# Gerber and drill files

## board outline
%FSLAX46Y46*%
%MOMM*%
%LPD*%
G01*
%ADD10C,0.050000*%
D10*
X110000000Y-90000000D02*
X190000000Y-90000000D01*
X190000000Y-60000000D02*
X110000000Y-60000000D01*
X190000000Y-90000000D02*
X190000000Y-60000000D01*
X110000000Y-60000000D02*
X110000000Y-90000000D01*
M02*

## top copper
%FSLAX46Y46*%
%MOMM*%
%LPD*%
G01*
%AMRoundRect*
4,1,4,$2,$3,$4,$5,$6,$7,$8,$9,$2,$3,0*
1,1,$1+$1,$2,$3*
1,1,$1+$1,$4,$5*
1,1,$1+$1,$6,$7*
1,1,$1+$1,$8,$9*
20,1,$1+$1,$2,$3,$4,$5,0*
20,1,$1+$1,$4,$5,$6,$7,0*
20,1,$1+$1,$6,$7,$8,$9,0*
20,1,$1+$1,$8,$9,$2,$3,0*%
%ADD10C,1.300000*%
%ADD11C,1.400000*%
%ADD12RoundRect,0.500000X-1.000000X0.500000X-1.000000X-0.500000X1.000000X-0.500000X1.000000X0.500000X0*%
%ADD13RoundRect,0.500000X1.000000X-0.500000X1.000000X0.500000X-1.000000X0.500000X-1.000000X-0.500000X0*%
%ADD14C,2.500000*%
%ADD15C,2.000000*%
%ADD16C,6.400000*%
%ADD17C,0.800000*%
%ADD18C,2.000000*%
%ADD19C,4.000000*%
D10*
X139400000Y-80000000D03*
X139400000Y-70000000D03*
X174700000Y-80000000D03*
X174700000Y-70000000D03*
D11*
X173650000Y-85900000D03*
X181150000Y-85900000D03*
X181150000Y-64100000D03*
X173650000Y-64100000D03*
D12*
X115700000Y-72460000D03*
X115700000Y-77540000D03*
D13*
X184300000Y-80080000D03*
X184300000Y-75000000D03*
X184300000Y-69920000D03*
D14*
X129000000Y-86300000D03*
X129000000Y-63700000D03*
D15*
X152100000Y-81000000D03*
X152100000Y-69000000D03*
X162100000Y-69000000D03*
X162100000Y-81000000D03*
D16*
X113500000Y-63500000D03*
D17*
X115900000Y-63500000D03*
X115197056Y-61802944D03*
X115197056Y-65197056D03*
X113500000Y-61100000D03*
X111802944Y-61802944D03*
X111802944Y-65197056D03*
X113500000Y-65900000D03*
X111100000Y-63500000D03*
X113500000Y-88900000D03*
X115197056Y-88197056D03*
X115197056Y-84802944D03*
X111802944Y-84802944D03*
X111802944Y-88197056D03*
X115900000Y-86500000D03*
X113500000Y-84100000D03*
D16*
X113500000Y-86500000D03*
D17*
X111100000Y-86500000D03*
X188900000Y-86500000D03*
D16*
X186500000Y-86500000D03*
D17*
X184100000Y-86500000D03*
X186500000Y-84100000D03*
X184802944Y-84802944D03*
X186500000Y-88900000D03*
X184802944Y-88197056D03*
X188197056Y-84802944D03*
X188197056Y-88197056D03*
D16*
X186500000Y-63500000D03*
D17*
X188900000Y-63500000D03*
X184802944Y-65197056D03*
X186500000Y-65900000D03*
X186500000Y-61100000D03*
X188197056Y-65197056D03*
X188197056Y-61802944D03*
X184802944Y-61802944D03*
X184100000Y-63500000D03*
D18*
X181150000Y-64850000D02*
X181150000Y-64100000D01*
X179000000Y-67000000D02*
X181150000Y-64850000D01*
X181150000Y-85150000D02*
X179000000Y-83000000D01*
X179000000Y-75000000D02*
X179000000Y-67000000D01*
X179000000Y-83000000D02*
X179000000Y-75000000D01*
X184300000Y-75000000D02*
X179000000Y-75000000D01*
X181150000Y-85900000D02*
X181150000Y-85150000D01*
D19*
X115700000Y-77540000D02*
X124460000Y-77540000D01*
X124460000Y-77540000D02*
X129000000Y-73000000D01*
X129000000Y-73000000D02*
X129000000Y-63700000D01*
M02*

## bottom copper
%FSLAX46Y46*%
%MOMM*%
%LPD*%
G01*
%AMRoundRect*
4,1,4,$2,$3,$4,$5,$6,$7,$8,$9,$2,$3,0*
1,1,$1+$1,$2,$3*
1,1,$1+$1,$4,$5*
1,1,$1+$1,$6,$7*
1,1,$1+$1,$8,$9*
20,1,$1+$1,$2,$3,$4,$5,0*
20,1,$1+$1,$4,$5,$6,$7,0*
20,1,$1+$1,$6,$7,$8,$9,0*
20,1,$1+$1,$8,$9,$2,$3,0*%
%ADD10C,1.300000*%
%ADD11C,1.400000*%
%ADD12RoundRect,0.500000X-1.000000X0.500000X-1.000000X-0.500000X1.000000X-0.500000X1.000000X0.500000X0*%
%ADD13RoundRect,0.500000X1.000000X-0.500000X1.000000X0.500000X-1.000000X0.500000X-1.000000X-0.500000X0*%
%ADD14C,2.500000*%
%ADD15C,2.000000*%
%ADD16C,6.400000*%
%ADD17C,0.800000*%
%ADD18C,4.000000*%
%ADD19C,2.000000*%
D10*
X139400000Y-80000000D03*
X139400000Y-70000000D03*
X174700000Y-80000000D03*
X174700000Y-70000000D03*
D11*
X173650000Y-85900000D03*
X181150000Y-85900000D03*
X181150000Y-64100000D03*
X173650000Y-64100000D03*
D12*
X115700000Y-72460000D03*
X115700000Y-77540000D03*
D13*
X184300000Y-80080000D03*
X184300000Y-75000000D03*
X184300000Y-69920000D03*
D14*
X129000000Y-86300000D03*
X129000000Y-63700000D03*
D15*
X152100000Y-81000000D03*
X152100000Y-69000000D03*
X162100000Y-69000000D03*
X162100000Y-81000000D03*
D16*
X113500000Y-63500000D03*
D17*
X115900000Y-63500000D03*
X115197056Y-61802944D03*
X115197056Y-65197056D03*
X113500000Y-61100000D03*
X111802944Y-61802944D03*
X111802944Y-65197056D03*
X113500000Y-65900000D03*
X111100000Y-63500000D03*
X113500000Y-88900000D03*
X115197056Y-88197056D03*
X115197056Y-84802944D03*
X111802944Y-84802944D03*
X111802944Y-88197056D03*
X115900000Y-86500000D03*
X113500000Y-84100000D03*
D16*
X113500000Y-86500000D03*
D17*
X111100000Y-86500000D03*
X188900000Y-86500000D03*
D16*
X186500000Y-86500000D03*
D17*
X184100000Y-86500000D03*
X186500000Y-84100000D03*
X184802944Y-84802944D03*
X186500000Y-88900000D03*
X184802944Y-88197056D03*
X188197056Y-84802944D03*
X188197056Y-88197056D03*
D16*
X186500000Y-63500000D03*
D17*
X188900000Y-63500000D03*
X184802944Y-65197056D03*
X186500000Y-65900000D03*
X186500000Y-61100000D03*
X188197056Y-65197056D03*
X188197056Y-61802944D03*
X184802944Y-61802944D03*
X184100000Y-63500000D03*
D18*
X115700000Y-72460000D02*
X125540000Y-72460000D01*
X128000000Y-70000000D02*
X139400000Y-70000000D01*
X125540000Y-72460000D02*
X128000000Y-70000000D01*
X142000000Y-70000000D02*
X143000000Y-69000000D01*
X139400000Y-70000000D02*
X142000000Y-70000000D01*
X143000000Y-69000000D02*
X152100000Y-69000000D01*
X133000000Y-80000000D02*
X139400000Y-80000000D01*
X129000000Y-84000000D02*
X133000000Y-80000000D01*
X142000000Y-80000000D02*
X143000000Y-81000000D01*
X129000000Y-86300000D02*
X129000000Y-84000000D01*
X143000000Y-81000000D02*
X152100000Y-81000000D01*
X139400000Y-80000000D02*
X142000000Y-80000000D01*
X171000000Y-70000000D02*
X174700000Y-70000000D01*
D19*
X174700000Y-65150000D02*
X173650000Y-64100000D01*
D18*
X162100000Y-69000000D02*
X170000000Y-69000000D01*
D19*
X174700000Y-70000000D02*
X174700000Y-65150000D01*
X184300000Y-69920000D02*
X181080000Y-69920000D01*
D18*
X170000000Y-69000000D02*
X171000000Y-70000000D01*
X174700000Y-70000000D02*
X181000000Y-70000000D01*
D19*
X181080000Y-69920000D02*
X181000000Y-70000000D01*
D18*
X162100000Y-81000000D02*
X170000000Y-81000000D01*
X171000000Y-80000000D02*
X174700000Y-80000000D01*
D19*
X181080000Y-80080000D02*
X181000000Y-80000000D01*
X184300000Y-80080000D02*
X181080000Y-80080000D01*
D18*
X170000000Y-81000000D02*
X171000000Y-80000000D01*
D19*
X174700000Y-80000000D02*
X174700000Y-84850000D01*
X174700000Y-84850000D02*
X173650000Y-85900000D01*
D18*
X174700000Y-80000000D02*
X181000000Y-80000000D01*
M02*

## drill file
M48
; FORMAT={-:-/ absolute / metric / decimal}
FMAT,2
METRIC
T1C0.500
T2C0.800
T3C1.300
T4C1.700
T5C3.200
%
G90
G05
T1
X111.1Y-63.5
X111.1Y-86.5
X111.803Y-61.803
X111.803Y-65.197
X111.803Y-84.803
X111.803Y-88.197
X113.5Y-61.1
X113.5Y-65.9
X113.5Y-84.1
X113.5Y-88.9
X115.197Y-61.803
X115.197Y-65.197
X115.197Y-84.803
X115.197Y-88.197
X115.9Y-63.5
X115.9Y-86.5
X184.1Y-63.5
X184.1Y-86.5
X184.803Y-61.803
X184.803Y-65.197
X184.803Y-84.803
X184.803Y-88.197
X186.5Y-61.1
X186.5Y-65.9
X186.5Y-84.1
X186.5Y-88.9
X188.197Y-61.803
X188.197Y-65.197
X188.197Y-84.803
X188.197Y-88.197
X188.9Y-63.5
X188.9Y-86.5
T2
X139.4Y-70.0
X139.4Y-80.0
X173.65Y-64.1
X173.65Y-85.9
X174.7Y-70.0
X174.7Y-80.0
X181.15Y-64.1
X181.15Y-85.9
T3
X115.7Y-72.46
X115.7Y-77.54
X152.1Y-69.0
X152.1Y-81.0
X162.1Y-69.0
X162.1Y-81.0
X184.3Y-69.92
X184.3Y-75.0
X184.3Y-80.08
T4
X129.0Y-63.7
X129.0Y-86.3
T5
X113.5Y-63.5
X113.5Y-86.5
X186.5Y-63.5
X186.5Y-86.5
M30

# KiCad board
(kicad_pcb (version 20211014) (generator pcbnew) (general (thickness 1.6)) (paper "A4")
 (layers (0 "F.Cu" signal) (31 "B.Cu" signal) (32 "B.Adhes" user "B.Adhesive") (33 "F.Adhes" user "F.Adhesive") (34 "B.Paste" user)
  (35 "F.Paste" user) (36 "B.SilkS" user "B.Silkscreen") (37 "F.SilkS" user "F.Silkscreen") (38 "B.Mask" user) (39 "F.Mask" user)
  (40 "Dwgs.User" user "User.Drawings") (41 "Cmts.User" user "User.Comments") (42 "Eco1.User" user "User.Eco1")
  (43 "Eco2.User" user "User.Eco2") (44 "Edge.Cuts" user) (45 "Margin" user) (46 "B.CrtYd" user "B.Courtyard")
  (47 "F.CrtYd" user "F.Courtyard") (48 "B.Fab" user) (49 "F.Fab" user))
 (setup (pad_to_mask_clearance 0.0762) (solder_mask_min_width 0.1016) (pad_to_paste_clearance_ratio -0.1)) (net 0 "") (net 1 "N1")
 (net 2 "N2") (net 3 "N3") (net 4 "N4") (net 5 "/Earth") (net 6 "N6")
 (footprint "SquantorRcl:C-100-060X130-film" (layer "F.Cu") (at 139.4 75 90)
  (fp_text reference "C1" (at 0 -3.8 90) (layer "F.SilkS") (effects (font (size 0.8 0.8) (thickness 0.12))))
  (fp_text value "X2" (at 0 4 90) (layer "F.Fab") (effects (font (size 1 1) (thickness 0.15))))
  (pad "1" thru_hole circle locked (at -5 0 90) (size 1.3 1.3) (drill 0.8) (layers *.Cu *.Mask) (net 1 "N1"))
  (pad "2" thru_hole circle locked (at 5 0 90) (size 1.3 1.3) (drill 0.8) (layers *.Cu *.Mask) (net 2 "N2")))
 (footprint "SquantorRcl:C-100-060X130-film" (layer "F.Cu") (at 174.7 75 90)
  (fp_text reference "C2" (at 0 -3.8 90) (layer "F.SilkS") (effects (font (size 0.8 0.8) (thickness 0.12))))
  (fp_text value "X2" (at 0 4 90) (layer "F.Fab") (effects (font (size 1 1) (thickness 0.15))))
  (pad "1" thru_hole circle locked (at -5 0 90) (size 1.3 1.3) (drill 0.8) (layers *.Cu *.Mask) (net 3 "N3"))
  (pad "2" thru_hole circle locked (at 5 0 90) (size 1.3 1.3) (drill 0.8) (layers *.Cu *.Mask) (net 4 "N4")))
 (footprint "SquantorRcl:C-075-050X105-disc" (layer "F.Cu") (at 177.4 85.9)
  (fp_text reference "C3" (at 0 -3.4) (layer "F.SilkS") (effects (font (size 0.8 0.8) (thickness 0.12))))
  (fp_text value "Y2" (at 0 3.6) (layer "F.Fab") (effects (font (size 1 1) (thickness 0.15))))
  (pad "1" thru_hole circle locked (at -3.75 0) (size 1.4 1.4) (drill 0.8) (layers *.Cu *.Mask) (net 3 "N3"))
  (pad "2" thru_hole circle locked (at 3.75 0) (size 1.4 1.4) (drill 0.8) (layers *.Cu *.Mask) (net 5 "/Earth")))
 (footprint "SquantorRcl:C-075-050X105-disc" (layer "F.Cu") (at 177.4 64.1 180)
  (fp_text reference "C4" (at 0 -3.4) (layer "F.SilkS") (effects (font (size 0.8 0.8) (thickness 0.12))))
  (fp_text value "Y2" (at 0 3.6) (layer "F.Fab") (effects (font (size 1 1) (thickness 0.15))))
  (pad "1" thru_hole circle locked (at -3.75 0 180) (size 1.4 1.4) (drill 0.8) (layers *.Cu *.Mask) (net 5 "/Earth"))
  (pad "2" thru_hole circle locked (at 3.75 0 180) (size 1.4 1.4) (drill 0.8) (layers *.Cu *.Mask) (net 4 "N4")))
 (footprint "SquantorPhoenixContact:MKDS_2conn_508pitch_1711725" (layer "F.Cu") (at 115.7 75 -90)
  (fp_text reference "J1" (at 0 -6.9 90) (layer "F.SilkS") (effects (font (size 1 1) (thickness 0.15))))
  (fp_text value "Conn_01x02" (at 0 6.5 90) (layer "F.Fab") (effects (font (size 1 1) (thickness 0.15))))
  (pad "1" thru_hole roundrect locked (at -2.54 0 270) (size 2 3) (drill 1.3) (layers *.Cu *.Mask) (roundrect_rratio 0.25) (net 2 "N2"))
  (pad "2" thru_hole roundrect locked (at 2.54 0 270) (size 2 3) (drill 1.3) (layers *.Cu *.Mask) (roundrect_rratio 0.25) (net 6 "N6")))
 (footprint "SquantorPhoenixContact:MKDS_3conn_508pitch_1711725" (layer "F.Cu") (at 184.3 75 90)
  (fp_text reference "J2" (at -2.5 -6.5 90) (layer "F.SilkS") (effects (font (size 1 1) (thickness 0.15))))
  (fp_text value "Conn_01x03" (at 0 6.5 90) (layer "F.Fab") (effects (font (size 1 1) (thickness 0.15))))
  (pad "1" thru_hole roundrect locked (at -5.08 0 90) (size 2 3) (drill 1.3) (layers *.Cu *.Mask) (roundrect_rratio 0.25) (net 3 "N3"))
  (pad "2" thru_hole roundrect locked (at 0 0 90) (size 2 3) (drill 1.3) (layers *.Cu *.Mask) (roundrect_rratio 0.25) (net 5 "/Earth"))
  (pad "3" thru_hole roundrect locked (at 5.08 0 90) (size 2 3) (drill 1.3) (layers *.Cu *.Mask) (roundrect_rratio 0.25) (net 4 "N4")))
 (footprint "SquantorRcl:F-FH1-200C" (layer "F.Cu") (at 129 75 90)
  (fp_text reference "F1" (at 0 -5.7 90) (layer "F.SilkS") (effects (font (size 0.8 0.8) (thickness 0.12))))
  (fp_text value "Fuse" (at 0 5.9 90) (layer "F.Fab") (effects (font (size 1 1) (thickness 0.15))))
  (pad "1" thru_hole circle locked (at -11.3 0 90) (size 2.5 2.5) (drill 1.7) (layers *.Cu *.Mask) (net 1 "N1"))
  (pad "2" thru_hole circle locked (at 11.3 0 90) (size 2.5 2.5) (drill 1.7) (layers *.Cu *.Mask) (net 6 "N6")))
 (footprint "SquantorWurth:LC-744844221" (layer "F.Cu") (at 157.1 75)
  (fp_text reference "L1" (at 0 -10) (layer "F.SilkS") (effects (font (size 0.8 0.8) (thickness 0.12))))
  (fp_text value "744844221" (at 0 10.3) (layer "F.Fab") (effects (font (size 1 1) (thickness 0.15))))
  (pad "1" thru_hole circle locked (at -5 6) (size 2 2) (drill 1.3) (layers *.Cu *.Mask) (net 1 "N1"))
  (pad "2" thru_hole circle locked (at -5 -6) (size 2 2) (drill 1.3) (layers *.Cu *.Mask) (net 2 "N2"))
  (pad "3" thru_hole circle locked (at 5 -6) (size 2 2) (drill 1.3) (layers *.Cu *.Mask) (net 4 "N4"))
  (pad "4" thru_hole circle locked (at 5 6) (size 2 2) (drill 1.3) (layers *.Cu *.Mask) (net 3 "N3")))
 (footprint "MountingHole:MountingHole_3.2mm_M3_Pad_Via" (layer "F.Cu") (at 113.5 63.5)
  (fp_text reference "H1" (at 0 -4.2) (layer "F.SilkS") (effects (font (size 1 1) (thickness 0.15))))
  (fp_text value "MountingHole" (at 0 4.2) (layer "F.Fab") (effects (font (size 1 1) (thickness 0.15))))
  (pad "1" thru_hole circle locked (at 0 0) (size 6.4 6.4) (drill 3.2) (layers *.Cu *.Mask))
  (pad "1" thru_hole circle locked (at 2.4 0) (size 0.8 0.8) (drill 0.5) (layers *.Cu *.Mask))
  (pad "1" thru_hole circle locked (at 1.697056 -1.697056) (size 0.8 0.8) (drill 0.5) (layers *.Cu *.Mask))
  (pad "1" thru_hole circle locked (at 1.697056 1.697056) (size 0.8 0.8) (drill 0.5) (layers *.Cu *.Mask))
  (pad "1" thru_hole circle locked (at 0 -2.4) (size 0.8 0.8) (drill 0.5) (layers *.Cu *.Mask))
  (pad "1" thru_hole circle locked (at -1.697056 -1.697056) (size 0.8 0.8) (drill 0.5) (layers *.Cu *.Mask))
  (pad "1" thru_hole circle locked (at -1.697056 1.697056) (size 0.8 0.8) (drill 0.5) (layers *.Cu *.Mask))
  (pad "1" thru_hole circle locked (at 0 2.4) (size 0.8 0.8) (drill 0.5) (layers *.Cu *.Mask))
  (pad "1" thru_hole circle locked (at -2.4 0) (size 0.8 0.8) (drill 0.5) (layers *.Cu *.Mask)))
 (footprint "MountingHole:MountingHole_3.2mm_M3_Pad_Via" (layer "F.Cu") (at 113.5 86.5)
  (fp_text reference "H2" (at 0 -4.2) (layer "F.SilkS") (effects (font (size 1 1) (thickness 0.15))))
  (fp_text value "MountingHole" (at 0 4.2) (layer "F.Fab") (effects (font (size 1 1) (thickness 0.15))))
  (pad "1" thru_hole circle locked (at 0 2.4) (size 0.8 0.8) (drill 0.5) (layers *.Cu *.Mask))
  (pad "1" thru_hole circle locked (at 1.697056 1.697056) (size 0.8 0.8) (drill 0.5) (layers *.Cu *.Mask))
  (pad "1" thru_hole circle locked (at 1.697056 -1.697056) (size 0.8 0.8) (drill 0.5) (layers *.Cu *.Mask))
  (pad "1" thru_hole circle locked (at -1.697056 -1.697056) (size 0.8 0.8) (drill 0.5) (layers *.Cu *.Mask))
  (pad "1" thru_hole circle locked (at -1.697056 1.697056) (size 0.8 0.8) (drill 0.5) (layers *.Cu *.Mask))
  (pad "1" thru_hole circle locked (at 2.4 0) (size 0.8 0.8) (drill 0.5) (layers *.Cu *.Mask))
  (pad "1" thru_hole circle locked (at 0 -2.4) (size 0.8 0.8) (drill 0.5) (layers *.Cu *.Mask))
  (pad "1" thru_hole circle locked (at 0 0) (size 6.4 6.4) (drill 3.2) (layers *.Cu *.Mask))
  (pad "1" thru_hole circle locked (at -2.4 0) (size 0.8 0.8) (drill 0.5) (layers *.Cu *.Mask)))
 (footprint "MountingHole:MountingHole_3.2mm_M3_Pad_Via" (layer "F.Cu") (at 186.5 86.5)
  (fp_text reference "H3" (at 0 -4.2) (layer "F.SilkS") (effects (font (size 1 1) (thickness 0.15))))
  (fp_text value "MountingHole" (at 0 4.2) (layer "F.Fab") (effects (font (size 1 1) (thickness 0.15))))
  (pad "1" thru_hole circle locked (at 2.4 0) (size 0.8 0.8) (drill 0.5) (layers *.Cu *.Mask))
  (pad "1" thru_hole circle locked (at 0 0) (size 6.4 6.4) (drill 3.2) (layers *.Cu *.Mask))
  (pad "1" thru_hole circle locked (at -2.4 0) (size 0.8 0.8) (drill 0.5) (layers *.Cu *.Mask))
  (pad "1" thru_hole circle locked (at 0 -2.4) (size 0.8 0.8) (drill 0.5) (layers *.Cu *.Mask))
  (pad "1" thru_hole circle locked (at -1.697056 -1.697056) (size 0.8 0.8) (drill 0.5) (layers *.Cu *.Mask))
  (pad "1" thru_hole circle locked (at 0 2.4) (size 0.8 0.8) (drill 0.5) (layers *.Cu *.Mask))
  (pad "1" thru_hole circle locked (at -1.697056 1.697056) (size 0.8 0.8) (drill 0.5) (layers *.Cu *.Mask))
  (pad "1" thru_hole circle locked (at 1.697056 -1.697056) (size 0.8 0.8) (drill 0.5) (layers *.Cu *.Mask))
  (pad "1" thru_hole circle locked (at 1.697056 1.697056) (size 0.8 0.8) (drill 0.5) (layers *.Cu *.Mask)))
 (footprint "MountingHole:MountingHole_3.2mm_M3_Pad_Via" (layer "F.Cu") (at 186.5 63.5)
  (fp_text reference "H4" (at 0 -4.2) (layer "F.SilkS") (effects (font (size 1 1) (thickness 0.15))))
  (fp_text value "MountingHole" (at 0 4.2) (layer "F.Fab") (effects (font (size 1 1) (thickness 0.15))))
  (pad "1" thru_hole circle locked (at 0 0) (size 6.4 6.4) (drill 3.2) (layers *.Cu *.Mask))
  (pad "1" thru_hole circle locked (at 2.4 0) (size 0.8 0.8) (drill 0.5) (layers *.Cu *.Mask))
  (pad "1" thru_hole circle locked (at -1.697056 1.697056) (size 0.8 0.8) (drill 0.5) (layers *.Cu *.Mask))
  (pad "1" thru_hole circle locked (at 0 2.4) (size 0.8 0.8) (drill 0.5) (layers *.Cu *.Mask))
  (pad "1" thru_hole circle locked (at 0 -2.4) (size 0.8 0.8) (drill 0.5) (layers *.Cu *.Mask))
  (pad "1" thru_hole circle locked (at 1.697056 1.697056) (size 0.8 0.8) (drill 0.5) (layers *.Cu *.Mask))
  (pad "1" thru_hole circle locked (at 1.697056 -1.697056) (size 0.8 0.8) (drill 0.5) (layers *.Cu *.Mask))
  (pad "1" thru_hole circle locked (at -1.697056 -1.697056) (size 0.8 0.8) (drill 0.5) (layers *.Cu *.Mask))
  (pad "1" thru_hole circle locked (at -2.4 0) (size 0.8 0.8) (drill 0.5) (layers *.Cu *.Mask)))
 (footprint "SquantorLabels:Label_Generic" (layer "B.Cu") (at 157.7 78.8 180)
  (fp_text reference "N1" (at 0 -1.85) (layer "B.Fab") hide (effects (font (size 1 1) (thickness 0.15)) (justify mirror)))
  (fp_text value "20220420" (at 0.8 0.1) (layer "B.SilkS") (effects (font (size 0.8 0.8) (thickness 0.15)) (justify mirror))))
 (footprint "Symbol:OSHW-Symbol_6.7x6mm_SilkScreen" (layer "B.Cu") (at 157 75 180)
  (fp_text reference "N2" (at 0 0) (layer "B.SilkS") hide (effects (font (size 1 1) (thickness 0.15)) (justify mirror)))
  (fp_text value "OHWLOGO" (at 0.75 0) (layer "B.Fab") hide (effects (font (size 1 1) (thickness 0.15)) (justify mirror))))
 (gr_line (start 110 90) (end 190 90) (layer "Edge.Cuts") (width 0.05))
 (gr_line (start 190 60) (end 110 60) (layer "Edge.Cuts") (width 0.05))
 (gr_line (start 190 90) (end 190 60) (layer "Edge.Cuts") (width 0.05))
 (gr_line (start 110 60) (end 110 90) (layer "Edge.Cuts") (width 0.05))
 (segment (start 115.7 72.46) (end 125.54 72.46) (width 4) (layer "B.Cu") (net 2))
 (segment (start 128 70) (end 139.4 70) (width 4) (layer "B.Cu") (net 2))
 (segment (start 125.54 72.46) (end 128 70) (width 4) (layer "B.Cu") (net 2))
 (segment (start 142 70) (end 143 69) (width 4) (layer "B.Cu") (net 2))
 (segment (start 139.4 70) (end 142 70) (width 4) (layer "B.Cu") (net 2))
 (segment (start 143 69) (end 152.1 69) (width 4) (layer "B.Cu") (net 2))
 (segment (start 133 80) (end 139.4 80) (width 4) (layer "B.Cu") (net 1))
 (segment (start 129 84) (end 133 80) (width 4) (layer "B.Cu") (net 1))
 (segment (start 142 80) (end 143 81) (width 4) (layer "B.Cu") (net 1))
 (segment (start 129 86.3) (end 129 84) (width 4) (layer "B.Cu") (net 1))
 (segment (start 143 81) (end 152.1 81) (width 4) (layer "B.Cu") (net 1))
 (segment (start 139.4 80) (end 142 80) (width 4) (layer "B.Cu") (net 1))
 (segment (start 171 70) (end 174.7 70) (width 4) (layer "B.Cu") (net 4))
 (segment (start 174.7 65.15) (end 173.65 64.1) (width 2) (layer "B.Cu") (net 4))
 (segment (start 162.1 69) (end 170 69) (width 4) (layer "B.Cu") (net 4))
 (segment (start 174.7 70) (end 174.7 65.15) (width 2) (layer "B.Cu") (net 4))
 (segment (start 184.3 69.92) (end 181.08 69.92) (width 2) (layer "B.Cu") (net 4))
 (segment (start 170 69) (end 171 70) (width 4) (layer "B.Cu") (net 4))
 (segment (start 174.7 70) (end 181 70) (width 4) (layer "B.Cu") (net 4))
 (segment (start 181.08 69.92) (end 181 70) (width 2) (layer "B.Cu") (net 4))
 (segment (start 162.1 81) (end 170 81) (width 4) (layer "B.Cu") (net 3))
 (segment (start 171 80) (end 174.7 80) (width 4) (layer "B.Cu") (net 3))
 (segment (start 181.08 80.08) (end 181 80) (width 2) (layer "B.Cu") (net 3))
 (segment (start 184.3 80.08) (end 181.08 80.08) (width 2) (layer "B.Cu") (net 3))
 (segment (start 170 81) (end 171 80) (width 4) (layer "B.Cu") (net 3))
 (segment (start 174.7 80) (end 174.7 84.85) (width 2) (layer "B.Cu") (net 3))
 (segment (start 174.7 84.85) (end 173.65 85.9) (width 2) (layer "B.Cu") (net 3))
 (segment (start 174.7 80) (end 181 80) (width 4) (layer "B.Cu") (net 3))
 (segment (start 181.15 64.85) (end 181.15 64.1) (width 2) (layer "F.Cu") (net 5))
 (segment (start 179 67) (end 181.15 64.85) (width 2) (layer "F.Cu") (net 5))
 (segment (start 181.15 85.15) (end 179 83) (width 2) (layer "F.Cu") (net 5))
 (segment (start 179 75) (end 179 67) (width 2) (layer "F.Cu") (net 5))
 (segment (start 179 83) (end 179 75) (width 2) (layer "F.Cu") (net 5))
 (segment (start 184.3 75) (end 179 75) (width 2) (layer "F.Cu") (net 5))
 (segment (start 181.15 85.9) (end 181.15 85.15) (width 2) (layer "F.Cu") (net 5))
 (segment (start 115.7 77.54) (end 124.46 77.54) (width 4) (layer "F.Cu") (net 6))
 (segment (start 124.46 77.54) (end 129 73) (width 4) (layer "F.Cu") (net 6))
 (segment (start 129 73) (end 129 63.7) (width 4) (layer "F.Cu") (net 6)))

